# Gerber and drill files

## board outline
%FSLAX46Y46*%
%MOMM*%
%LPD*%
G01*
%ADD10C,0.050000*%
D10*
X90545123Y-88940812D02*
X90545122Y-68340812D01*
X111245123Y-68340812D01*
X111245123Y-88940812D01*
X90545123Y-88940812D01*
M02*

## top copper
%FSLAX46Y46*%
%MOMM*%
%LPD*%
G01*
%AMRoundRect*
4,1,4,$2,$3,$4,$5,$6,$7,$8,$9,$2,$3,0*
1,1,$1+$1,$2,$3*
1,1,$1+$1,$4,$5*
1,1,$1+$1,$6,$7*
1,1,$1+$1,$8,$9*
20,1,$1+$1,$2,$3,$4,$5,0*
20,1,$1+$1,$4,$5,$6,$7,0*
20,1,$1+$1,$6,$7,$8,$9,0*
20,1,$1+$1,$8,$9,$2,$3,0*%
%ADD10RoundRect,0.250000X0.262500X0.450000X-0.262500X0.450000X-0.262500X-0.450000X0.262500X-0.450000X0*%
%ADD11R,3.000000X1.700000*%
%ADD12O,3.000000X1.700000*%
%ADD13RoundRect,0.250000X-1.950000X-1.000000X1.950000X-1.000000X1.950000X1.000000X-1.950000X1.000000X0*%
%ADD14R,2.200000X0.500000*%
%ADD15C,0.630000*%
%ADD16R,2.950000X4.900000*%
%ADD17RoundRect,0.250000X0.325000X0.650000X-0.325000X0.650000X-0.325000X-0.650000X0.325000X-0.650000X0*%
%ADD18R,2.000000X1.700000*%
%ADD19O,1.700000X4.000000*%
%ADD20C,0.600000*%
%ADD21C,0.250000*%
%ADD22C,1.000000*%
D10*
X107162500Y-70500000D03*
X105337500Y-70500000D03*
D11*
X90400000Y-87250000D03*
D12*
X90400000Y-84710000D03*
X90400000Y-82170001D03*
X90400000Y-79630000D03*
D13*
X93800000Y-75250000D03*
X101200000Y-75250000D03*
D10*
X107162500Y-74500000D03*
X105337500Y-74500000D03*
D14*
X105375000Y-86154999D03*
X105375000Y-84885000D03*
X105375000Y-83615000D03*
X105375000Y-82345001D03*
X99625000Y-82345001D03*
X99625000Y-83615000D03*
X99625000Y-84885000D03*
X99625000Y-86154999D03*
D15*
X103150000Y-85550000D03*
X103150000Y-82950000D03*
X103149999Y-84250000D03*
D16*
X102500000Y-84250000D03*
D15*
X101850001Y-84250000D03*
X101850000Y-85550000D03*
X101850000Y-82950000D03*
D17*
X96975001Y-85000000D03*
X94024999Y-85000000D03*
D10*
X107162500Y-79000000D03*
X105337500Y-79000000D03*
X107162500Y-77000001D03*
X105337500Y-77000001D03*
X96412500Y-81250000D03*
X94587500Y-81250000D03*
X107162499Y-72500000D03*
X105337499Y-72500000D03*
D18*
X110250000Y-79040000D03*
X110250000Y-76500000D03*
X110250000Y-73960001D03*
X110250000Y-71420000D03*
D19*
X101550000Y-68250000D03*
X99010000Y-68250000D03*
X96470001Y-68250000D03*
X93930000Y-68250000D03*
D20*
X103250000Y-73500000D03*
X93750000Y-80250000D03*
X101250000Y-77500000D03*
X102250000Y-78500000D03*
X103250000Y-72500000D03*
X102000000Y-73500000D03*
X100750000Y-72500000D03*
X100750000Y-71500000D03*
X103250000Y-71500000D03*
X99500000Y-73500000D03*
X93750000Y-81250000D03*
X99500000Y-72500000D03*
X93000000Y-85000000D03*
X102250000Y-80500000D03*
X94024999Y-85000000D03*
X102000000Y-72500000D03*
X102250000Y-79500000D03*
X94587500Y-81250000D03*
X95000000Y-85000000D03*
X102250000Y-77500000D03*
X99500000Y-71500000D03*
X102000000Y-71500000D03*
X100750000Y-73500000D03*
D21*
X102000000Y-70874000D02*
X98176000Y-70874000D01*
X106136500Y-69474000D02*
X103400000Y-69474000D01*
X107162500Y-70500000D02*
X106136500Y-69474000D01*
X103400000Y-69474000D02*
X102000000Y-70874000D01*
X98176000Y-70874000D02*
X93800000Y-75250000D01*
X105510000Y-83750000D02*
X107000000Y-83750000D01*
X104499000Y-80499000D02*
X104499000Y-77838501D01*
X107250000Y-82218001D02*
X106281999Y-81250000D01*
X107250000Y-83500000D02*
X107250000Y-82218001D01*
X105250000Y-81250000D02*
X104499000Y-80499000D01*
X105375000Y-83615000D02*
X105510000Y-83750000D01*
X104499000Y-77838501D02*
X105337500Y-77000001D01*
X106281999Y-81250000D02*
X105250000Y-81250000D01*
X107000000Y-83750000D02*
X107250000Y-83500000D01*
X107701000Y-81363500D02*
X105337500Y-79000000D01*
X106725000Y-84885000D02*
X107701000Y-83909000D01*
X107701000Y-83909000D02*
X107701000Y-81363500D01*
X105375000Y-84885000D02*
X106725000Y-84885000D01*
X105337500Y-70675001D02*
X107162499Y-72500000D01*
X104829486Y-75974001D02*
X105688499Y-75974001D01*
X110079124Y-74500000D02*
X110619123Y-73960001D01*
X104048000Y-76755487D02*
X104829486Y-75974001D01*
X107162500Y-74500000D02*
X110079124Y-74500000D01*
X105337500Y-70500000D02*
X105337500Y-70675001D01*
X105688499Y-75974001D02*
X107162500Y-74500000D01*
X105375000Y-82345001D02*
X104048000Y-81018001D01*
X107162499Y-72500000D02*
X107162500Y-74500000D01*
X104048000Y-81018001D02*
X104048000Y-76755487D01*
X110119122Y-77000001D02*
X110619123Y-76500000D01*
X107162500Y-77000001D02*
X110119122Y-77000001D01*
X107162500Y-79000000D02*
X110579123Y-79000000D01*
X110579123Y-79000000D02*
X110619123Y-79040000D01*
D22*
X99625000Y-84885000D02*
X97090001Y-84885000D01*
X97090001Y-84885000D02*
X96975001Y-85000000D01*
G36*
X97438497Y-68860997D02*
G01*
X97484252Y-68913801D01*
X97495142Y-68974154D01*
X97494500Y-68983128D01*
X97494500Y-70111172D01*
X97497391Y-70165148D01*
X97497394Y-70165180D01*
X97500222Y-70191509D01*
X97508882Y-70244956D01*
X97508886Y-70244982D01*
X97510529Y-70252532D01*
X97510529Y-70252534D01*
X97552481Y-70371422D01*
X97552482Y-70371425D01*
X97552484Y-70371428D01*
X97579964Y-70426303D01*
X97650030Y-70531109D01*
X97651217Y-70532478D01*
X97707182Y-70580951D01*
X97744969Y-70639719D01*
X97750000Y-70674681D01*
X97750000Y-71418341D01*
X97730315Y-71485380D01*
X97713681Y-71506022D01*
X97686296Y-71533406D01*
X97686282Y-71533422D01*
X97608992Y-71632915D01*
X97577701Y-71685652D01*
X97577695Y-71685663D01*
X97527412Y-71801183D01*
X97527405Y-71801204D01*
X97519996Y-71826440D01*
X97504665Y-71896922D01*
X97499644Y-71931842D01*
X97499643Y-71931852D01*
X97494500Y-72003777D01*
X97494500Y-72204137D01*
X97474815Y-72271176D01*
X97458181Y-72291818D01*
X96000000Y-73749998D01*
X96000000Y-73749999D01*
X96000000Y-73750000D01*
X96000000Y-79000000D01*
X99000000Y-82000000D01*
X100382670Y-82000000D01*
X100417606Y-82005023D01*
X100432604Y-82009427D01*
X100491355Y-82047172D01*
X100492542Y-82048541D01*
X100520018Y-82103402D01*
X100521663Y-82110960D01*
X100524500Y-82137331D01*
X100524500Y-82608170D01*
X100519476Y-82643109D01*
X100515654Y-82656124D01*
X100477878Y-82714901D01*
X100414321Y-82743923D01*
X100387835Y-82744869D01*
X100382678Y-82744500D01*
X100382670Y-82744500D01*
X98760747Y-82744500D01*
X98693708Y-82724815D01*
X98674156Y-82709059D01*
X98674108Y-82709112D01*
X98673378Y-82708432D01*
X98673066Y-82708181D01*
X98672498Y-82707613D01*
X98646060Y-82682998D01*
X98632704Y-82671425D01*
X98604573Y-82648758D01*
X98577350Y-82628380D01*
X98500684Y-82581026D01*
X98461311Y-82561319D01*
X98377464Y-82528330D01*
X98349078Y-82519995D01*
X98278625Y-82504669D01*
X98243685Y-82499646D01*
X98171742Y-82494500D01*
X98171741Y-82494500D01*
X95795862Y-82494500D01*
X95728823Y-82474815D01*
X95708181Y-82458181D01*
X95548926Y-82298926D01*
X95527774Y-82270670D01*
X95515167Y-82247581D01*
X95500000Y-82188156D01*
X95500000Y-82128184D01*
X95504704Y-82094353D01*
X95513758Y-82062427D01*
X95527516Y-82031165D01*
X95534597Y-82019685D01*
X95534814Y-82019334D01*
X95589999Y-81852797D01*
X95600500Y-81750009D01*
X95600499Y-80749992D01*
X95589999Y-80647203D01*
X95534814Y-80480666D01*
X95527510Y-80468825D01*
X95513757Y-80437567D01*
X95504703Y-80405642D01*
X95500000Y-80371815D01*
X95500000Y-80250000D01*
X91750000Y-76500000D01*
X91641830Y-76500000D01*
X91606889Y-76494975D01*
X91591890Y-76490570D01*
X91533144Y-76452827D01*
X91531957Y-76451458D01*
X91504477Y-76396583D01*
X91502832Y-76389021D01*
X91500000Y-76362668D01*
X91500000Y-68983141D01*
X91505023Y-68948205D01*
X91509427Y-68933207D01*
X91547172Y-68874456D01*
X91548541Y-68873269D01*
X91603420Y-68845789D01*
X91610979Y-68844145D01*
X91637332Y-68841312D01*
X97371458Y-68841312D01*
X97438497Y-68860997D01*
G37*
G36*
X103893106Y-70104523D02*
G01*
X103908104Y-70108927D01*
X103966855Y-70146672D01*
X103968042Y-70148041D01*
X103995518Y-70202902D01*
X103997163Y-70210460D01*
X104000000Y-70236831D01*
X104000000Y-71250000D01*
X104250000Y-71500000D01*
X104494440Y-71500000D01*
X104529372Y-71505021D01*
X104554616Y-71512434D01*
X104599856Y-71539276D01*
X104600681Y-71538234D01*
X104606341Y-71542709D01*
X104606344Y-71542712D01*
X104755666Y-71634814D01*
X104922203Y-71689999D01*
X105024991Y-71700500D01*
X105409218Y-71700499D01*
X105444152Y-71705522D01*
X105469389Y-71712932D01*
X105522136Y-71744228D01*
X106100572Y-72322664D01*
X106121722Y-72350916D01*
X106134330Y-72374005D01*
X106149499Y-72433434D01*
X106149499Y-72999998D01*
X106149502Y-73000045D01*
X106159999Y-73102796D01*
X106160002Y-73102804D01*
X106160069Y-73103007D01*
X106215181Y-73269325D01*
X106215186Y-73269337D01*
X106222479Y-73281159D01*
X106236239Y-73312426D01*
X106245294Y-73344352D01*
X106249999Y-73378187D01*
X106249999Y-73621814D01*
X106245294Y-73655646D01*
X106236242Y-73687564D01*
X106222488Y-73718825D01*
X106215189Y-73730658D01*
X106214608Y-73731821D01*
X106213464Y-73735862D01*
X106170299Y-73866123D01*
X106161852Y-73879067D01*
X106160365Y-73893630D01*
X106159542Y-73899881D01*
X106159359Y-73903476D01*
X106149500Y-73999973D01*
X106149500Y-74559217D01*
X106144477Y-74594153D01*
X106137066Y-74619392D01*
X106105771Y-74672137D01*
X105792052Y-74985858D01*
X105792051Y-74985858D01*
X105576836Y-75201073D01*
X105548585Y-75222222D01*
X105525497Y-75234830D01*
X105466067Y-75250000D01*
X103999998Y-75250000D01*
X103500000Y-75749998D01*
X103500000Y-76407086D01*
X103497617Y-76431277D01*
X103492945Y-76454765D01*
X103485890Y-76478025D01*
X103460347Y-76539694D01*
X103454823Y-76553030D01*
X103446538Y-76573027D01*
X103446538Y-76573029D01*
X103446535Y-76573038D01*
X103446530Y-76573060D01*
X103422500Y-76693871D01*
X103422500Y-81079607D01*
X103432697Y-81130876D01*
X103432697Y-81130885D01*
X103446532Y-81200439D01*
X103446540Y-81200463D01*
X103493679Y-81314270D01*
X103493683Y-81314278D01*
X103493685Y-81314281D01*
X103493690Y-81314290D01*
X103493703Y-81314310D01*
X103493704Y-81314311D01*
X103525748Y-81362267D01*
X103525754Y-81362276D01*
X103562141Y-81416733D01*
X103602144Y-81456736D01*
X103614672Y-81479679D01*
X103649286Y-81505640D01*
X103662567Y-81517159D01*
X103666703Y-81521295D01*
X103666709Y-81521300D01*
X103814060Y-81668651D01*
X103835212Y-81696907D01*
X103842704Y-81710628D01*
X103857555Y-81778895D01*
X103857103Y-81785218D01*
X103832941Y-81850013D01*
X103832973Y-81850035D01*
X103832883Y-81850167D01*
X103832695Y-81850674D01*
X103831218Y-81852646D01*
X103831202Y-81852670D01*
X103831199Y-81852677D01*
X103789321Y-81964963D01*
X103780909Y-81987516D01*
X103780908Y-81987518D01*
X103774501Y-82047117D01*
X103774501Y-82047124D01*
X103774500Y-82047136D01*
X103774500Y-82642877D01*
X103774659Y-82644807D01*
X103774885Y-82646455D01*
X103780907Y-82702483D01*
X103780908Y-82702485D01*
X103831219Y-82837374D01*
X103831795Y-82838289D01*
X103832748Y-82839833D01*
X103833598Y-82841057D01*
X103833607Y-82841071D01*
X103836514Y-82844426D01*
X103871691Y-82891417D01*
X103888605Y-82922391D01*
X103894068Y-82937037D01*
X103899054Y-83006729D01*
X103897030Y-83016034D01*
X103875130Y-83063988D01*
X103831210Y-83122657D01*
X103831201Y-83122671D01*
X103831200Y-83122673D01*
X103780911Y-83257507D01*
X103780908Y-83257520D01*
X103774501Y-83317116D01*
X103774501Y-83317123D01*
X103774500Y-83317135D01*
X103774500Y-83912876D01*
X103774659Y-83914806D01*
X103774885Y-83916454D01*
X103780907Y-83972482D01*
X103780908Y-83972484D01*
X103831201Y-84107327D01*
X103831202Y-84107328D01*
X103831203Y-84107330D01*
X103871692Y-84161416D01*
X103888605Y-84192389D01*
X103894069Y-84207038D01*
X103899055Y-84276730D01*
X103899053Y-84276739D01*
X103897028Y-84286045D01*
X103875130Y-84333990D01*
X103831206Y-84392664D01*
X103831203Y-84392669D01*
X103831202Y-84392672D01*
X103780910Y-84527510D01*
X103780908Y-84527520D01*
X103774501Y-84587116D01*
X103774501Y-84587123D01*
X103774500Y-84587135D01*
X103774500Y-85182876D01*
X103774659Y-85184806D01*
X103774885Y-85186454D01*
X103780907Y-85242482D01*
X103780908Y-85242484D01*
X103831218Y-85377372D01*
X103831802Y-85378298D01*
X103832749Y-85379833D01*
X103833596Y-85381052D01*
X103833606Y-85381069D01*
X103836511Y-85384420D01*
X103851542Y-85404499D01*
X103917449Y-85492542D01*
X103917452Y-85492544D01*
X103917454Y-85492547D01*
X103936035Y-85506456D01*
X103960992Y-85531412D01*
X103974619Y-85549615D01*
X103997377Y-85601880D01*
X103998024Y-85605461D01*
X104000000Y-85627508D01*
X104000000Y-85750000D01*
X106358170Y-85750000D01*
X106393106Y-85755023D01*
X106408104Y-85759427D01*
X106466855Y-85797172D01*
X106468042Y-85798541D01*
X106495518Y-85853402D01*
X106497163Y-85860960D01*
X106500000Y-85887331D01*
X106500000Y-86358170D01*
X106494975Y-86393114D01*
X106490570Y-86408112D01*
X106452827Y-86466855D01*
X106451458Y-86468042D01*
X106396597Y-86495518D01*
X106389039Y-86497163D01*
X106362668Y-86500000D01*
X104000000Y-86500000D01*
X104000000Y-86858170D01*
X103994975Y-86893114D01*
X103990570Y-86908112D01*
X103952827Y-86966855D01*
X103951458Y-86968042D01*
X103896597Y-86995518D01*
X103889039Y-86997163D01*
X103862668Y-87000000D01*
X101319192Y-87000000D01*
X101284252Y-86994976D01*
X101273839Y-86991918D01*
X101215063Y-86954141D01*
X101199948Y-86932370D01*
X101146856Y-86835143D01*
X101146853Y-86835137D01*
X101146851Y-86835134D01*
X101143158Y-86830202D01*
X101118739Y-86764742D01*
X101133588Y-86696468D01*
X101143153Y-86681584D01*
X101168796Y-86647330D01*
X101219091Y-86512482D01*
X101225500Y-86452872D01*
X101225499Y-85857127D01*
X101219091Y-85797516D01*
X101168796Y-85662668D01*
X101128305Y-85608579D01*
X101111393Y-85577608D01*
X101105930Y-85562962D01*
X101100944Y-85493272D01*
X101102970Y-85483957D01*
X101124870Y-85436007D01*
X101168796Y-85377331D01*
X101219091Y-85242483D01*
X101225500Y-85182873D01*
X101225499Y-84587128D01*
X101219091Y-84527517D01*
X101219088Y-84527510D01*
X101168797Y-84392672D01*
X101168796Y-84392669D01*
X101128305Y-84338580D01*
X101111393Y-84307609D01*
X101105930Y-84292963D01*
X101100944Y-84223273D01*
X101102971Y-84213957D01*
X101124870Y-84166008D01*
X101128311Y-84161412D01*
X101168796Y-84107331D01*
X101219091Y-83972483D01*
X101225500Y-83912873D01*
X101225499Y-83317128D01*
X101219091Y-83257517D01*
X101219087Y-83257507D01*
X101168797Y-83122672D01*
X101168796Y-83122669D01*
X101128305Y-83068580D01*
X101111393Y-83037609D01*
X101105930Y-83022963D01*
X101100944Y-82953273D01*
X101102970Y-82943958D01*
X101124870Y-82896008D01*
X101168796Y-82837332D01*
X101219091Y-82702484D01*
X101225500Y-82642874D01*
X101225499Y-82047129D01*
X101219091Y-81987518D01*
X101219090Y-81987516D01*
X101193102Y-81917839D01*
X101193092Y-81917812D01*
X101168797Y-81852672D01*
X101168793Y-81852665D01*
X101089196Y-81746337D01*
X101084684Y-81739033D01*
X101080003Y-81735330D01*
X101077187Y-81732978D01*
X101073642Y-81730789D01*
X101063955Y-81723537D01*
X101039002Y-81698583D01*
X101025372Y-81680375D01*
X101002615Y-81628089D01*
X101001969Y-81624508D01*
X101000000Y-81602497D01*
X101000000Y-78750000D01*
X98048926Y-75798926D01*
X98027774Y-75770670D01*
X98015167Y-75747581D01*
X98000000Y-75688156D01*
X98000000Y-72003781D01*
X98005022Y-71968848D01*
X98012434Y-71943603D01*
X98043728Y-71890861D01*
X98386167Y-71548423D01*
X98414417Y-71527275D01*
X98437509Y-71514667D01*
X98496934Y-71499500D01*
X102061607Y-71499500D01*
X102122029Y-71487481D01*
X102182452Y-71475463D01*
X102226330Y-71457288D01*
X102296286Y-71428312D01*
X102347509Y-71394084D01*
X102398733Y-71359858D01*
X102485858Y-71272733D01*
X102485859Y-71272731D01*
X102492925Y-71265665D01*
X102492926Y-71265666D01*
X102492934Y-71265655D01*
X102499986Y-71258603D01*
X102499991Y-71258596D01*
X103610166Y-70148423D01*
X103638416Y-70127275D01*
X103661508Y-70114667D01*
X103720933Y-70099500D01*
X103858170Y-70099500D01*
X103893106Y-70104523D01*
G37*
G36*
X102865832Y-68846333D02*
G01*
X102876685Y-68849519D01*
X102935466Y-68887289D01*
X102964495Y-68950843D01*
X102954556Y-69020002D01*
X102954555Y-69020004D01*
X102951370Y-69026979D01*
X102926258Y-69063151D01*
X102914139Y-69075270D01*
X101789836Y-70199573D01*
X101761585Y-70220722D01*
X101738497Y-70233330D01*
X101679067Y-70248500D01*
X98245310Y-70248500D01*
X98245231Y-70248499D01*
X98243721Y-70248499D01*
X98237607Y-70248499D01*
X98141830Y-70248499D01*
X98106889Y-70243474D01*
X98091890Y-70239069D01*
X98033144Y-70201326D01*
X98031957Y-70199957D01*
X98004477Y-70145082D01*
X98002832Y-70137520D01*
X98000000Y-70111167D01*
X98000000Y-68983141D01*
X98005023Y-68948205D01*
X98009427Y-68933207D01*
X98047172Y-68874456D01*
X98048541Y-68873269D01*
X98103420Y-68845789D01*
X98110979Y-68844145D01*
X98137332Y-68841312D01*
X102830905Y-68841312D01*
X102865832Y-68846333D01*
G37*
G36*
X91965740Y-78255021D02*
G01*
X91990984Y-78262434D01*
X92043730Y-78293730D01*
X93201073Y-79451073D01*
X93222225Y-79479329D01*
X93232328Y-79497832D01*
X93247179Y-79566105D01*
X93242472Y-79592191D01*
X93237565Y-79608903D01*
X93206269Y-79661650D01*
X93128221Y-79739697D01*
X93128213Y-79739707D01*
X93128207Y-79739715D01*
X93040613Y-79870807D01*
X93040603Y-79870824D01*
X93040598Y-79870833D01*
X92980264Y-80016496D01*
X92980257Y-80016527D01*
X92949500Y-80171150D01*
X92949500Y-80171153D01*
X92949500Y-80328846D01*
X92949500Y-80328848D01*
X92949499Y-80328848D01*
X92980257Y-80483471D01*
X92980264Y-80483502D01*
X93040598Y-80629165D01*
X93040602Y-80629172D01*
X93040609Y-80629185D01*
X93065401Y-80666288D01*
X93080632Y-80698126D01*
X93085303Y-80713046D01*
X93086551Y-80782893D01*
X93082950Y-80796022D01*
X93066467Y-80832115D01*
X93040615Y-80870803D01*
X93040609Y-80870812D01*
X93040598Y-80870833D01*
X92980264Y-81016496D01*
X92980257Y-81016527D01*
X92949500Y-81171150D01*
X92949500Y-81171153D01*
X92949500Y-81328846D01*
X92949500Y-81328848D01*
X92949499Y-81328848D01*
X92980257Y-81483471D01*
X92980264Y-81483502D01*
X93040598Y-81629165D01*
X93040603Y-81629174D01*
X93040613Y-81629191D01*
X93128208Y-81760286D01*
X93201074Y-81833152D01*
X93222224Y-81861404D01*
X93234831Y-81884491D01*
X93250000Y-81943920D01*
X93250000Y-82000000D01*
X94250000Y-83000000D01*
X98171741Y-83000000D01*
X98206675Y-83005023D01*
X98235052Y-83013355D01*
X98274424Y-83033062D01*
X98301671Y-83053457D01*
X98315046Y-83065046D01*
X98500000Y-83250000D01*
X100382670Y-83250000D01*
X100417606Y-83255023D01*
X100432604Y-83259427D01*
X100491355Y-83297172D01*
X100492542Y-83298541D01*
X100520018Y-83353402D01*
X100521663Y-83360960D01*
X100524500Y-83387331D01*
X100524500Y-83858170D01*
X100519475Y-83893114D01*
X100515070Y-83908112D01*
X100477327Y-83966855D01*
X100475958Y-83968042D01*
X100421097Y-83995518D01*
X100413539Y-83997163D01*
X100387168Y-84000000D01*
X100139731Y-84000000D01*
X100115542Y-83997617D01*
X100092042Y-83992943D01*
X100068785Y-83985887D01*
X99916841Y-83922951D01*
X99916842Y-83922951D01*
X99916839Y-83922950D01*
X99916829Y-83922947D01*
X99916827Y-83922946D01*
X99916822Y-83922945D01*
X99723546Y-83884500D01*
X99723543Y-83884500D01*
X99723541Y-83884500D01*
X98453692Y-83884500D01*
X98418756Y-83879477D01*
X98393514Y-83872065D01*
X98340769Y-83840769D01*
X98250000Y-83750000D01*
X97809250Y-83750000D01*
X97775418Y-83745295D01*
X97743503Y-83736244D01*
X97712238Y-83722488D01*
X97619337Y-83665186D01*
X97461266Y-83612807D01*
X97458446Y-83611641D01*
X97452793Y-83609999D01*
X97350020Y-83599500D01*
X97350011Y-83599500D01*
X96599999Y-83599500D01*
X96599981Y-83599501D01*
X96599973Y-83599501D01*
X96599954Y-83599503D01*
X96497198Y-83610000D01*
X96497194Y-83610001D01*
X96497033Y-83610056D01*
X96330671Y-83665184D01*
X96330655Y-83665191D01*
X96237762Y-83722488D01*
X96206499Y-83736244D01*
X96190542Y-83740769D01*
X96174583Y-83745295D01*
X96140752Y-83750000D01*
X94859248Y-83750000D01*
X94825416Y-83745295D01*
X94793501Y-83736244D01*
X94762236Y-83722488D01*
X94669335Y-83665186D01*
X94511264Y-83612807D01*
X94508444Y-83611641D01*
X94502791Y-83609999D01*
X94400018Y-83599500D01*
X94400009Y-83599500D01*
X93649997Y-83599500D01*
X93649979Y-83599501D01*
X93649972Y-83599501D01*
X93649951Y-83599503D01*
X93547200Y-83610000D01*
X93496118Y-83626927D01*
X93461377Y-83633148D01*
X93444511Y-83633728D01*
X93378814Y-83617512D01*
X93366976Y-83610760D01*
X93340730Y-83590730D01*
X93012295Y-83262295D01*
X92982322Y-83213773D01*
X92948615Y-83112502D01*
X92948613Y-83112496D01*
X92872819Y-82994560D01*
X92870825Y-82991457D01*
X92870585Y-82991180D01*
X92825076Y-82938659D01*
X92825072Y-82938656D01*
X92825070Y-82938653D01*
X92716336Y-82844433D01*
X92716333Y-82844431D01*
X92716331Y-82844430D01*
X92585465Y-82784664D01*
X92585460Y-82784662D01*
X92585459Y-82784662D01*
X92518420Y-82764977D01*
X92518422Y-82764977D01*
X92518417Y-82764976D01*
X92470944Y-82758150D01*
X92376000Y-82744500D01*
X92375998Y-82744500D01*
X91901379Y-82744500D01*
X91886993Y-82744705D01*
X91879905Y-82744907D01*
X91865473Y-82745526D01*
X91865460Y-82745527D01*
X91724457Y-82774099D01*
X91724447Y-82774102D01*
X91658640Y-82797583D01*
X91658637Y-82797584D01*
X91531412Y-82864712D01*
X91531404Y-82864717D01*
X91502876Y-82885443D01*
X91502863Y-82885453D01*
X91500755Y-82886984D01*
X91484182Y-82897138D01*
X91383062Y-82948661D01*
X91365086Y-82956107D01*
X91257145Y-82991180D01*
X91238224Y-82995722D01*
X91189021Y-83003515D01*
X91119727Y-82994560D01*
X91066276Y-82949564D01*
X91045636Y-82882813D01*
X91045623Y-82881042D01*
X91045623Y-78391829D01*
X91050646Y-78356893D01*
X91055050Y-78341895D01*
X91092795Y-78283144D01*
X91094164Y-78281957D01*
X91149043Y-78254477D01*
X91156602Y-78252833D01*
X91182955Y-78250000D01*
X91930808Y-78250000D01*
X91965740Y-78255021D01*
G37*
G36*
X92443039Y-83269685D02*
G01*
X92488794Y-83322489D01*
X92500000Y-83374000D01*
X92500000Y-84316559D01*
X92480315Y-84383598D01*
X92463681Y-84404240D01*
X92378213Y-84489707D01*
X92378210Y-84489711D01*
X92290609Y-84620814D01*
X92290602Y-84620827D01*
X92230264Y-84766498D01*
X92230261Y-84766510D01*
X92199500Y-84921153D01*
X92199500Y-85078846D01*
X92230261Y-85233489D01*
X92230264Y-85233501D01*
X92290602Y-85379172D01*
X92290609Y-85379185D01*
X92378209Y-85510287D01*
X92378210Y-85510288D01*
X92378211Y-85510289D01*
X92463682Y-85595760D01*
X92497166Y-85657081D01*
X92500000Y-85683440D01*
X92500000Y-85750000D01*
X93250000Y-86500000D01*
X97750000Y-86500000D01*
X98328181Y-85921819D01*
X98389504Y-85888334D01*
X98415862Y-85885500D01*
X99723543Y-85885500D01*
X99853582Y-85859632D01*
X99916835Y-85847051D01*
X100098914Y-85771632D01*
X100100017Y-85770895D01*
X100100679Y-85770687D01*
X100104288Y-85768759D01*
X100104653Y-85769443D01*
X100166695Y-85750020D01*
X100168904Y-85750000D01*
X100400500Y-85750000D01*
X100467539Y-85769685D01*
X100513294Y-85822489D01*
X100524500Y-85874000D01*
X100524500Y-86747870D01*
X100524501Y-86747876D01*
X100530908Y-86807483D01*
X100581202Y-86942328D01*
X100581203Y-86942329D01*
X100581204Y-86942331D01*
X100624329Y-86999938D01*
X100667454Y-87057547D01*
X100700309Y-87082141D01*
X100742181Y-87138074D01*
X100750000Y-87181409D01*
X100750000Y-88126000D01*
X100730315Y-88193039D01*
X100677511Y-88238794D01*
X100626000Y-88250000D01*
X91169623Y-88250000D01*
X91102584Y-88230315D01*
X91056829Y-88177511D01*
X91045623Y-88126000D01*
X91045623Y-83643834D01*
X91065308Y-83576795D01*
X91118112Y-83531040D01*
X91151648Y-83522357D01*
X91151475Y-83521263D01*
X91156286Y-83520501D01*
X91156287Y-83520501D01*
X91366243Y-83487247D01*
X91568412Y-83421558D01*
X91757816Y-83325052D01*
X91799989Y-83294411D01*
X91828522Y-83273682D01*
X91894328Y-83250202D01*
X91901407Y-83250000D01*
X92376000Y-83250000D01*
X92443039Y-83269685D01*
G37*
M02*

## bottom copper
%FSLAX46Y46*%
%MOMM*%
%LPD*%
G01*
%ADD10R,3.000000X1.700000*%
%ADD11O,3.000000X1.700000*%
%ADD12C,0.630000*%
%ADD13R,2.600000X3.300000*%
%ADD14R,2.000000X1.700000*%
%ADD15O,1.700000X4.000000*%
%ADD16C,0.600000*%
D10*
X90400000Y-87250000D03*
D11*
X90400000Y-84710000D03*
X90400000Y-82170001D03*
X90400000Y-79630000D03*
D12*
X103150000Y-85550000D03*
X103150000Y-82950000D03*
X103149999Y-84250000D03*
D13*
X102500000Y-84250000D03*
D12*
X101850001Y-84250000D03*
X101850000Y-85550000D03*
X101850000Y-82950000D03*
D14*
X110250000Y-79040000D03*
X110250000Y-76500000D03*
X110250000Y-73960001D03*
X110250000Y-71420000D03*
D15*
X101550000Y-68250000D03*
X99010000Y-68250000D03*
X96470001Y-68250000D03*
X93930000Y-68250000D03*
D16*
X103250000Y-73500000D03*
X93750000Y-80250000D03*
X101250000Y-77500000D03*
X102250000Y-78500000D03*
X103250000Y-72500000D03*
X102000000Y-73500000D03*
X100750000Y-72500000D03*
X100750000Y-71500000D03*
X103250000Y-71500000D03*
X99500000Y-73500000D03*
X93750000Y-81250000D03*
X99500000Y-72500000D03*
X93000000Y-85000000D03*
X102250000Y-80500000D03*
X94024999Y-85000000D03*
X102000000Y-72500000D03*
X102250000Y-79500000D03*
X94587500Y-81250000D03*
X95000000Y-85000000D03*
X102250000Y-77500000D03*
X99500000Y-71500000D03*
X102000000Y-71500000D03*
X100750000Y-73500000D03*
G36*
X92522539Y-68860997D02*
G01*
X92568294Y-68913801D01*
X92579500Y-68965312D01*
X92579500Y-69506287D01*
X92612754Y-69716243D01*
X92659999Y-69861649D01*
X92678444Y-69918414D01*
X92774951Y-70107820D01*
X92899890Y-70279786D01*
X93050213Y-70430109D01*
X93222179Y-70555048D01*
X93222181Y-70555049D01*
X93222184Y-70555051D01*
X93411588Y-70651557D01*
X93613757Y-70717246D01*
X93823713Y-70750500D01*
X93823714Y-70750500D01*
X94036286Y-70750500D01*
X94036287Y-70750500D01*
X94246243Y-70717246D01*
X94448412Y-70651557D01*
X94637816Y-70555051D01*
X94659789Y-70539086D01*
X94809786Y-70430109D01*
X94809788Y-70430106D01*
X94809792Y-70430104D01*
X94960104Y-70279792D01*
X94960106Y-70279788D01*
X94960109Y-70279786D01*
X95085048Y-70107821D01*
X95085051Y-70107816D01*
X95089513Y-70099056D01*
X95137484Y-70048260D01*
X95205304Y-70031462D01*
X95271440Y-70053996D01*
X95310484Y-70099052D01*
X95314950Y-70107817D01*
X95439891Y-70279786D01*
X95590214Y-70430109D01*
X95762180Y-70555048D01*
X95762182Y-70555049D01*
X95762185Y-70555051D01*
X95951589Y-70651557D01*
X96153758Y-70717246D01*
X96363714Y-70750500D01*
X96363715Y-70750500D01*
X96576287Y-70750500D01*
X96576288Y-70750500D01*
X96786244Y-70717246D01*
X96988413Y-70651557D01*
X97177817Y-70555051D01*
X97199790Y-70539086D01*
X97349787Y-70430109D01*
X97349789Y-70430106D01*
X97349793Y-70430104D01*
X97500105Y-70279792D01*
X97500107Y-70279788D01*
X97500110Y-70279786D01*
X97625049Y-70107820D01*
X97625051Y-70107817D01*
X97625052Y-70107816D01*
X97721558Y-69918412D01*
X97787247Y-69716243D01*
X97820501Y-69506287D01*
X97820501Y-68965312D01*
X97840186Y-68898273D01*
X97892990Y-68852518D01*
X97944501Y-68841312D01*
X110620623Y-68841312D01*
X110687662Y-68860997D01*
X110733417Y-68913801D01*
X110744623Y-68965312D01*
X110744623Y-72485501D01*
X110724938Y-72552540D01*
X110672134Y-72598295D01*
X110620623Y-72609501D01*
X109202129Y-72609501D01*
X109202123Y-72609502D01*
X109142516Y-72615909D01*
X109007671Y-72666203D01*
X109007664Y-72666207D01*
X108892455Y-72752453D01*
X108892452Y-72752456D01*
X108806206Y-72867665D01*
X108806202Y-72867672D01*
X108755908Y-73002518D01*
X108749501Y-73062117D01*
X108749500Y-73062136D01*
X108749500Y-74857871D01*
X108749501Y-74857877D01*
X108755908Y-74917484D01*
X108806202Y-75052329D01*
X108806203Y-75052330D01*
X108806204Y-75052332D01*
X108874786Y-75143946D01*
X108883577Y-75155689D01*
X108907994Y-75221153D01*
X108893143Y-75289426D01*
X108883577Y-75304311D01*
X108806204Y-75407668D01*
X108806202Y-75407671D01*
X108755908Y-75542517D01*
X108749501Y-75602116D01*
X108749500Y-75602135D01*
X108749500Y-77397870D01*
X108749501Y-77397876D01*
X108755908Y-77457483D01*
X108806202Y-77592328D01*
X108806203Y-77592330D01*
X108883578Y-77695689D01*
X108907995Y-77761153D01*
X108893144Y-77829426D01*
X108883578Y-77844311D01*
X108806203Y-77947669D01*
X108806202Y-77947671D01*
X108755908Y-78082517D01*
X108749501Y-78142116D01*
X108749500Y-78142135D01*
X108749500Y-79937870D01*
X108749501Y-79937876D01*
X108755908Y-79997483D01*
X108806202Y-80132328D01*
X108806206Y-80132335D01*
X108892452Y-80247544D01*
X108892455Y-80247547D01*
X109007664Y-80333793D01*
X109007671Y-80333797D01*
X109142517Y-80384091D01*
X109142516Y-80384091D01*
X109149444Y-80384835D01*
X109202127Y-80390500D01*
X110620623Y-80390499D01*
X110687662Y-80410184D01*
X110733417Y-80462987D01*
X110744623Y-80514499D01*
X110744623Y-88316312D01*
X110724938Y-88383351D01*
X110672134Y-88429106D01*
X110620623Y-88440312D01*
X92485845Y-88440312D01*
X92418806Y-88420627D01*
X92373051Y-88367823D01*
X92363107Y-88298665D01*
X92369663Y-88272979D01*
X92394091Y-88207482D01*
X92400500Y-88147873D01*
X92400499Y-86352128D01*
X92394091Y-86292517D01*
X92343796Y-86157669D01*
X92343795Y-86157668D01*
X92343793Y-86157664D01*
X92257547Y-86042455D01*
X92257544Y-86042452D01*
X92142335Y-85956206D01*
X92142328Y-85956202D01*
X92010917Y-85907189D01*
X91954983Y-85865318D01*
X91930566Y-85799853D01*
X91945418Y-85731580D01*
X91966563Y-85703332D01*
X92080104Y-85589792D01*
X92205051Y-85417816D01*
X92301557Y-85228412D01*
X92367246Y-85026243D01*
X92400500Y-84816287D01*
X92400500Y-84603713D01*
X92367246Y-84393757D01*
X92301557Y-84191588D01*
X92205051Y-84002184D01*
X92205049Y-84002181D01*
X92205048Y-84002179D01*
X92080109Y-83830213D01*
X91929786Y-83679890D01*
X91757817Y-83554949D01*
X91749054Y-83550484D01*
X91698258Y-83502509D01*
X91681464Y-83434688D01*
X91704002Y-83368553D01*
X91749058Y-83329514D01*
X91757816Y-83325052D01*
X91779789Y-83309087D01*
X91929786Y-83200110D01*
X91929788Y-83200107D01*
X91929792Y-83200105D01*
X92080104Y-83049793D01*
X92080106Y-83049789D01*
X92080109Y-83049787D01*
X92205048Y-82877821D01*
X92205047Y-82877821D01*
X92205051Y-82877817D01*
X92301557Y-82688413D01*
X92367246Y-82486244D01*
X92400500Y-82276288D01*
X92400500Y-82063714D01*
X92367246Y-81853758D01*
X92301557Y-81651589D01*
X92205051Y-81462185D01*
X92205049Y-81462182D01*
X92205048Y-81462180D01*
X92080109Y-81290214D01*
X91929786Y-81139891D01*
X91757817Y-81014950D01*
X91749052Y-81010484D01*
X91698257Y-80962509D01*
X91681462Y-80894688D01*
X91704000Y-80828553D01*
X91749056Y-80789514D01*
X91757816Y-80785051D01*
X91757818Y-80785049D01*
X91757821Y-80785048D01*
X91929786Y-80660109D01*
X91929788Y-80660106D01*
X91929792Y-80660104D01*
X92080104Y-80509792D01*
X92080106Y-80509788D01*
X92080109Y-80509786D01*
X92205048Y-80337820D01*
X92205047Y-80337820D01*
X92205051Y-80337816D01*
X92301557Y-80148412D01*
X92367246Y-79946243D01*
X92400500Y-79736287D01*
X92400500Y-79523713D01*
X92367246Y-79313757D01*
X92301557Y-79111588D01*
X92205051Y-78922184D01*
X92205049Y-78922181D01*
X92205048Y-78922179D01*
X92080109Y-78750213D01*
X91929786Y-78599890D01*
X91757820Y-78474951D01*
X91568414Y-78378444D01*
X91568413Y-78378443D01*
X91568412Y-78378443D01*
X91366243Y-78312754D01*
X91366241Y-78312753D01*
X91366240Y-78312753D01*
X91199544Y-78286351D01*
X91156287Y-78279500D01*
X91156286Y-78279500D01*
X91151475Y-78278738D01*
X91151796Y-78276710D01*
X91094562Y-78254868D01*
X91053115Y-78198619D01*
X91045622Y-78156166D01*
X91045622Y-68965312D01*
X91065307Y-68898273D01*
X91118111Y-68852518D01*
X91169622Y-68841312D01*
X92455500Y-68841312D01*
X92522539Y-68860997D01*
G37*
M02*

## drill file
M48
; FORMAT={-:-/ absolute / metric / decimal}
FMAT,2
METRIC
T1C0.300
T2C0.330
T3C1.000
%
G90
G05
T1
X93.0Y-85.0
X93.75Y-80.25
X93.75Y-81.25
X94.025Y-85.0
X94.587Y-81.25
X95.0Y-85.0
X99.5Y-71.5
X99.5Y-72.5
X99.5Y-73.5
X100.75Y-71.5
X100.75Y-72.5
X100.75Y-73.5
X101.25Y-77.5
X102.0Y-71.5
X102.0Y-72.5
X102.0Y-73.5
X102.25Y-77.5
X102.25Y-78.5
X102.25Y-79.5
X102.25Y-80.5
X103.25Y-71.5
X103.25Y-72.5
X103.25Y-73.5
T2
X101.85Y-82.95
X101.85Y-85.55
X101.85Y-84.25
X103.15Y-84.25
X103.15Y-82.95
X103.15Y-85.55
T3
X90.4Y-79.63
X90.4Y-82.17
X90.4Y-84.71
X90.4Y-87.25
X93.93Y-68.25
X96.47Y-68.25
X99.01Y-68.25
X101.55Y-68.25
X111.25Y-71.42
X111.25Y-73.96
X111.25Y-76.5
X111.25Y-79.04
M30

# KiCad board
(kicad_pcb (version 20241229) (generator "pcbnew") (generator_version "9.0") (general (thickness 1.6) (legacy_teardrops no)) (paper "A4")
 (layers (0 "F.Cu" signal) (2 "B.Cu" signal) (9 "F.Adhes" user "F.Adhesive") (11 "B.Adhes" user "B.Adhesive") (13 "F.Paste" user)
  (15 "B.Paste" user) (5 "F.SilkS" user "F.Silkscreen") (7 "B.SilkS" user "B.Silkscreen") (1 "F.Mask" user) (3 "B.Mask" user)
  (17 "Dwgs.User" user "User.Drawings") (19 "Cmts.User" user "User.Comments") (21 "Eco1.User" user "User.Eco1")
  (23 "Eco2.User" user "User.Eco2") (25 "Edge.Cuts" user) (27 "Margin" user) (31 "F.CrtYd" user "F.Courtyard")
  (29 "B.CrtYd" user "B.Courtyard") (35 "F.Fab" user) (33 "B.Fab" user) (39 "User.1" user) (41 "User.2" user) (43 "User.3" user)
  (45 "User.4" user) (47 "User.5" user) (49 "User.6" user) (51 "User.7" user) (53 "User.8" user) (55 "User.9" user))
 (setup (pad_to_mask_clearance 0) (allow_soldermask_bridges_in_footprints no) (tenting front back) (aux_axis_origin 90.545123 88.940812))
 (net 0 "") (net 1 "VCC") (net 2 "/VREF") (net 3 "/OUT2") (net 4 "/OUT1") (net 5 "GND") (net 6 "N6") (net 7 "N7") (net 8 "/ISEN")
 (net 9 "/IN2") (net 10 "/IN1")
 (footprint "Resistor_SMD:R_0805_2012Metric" (layer "F.Cu") (at 106.25 70.5 180)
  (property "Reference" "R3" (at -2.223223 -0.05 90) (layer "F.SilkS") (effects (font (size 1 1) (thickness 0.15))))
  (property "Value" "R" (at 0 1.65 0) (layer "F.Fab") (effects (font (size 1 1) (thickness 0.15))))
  (pad "1" smd roundrect (at -0.9125 0 180) (size 1.025 1.4) (layers "F.Cu" "F.Mask" "F.Paste") (roundrect_rratio 0.243902) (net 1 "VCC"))
  (pad "2" smd roundrect (at 0.9125 0 180) (size 1.025 1.4) (layers "F.Cu" "F.Mask" "F.Paste") (roundrect_rratio 0.243902) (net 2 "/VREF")))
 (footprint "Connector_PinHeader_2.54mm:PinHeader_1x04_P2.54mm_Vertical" (layer "F.Cu") (at 90.4 87.25 180)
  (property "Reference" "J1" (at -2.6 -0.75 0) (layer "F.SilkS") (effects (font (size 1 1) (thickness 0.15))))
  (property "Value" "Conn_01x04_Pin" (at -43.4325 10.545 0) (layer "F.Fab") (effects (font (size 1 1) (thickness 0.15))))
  (pad "1" thru_hole rect (at 0 0 180) (size 3 1.7) (drill 1) (layers "*.Cu" "*.Mask") (remove_unused_layers no) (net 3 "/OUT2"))
  (pad "2" thru_hole oval (at 0 2.54 180) (size 3 1.7) (drill 1) (layers "*.Cu" "*.Mask") (remove_unused_layers no) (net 3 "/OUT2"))
  (pad "3" thru_hole oval (at 0 5.079999 180) (size 3 1.7) (drill 1) (layers "*.Cu" "*.Mask") (remove_unused_layers no) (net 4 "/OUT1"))
  (pad "4" thru_hole oval (at 0 7.62 180) (size 3 1.7) (drill 1) (layers "*.Cu" "*.Mask") (remove_unused_layers no) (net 4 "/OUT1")))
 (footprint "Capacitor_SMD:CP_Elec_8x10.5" (layer "F.Cu") (at 97.5 75.25)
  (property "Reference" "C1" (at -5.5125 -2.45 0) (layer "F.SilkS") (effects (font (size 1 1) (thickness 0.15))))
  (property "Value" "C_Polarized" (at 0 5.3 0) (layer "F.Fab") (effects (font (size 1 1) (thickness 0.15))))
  (pad "1" smd roundrect (at -3.7 0) (size 4.4 2.5) (layers "F.Cu" "F.Mask" "F.Paste") (roundrect_rratio 0.1) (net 1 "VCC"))
  (pad "2" smd roundrect (at 3.7 0) (size 4.4 2.5) (layers "F.Cu" "F.Mask" "F.Paste") (roundrect_rratio 0.1) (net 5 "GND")))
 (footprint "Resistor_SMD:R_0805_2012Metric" (layer "F.Cu") (at 106.25 74.5 180)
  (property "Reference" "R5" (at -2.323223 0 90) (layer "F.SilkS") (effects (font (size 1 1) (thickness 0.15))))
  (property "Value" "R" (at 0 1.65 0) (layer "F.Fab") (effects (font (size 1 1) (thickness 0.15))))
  (pad "1" smd roundrect (at -0.9125 0 180) (size 1.025 1.4) (layers "F.Cu" "F.Mask" "F.Paste") (roundrect_rratio 0.243902) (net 2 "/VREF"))
  (pad "2" smd roundrect (at 0.9125 0 180) (size 1.025 1.4) (layers "F.Cu" "F.Mask" "F.Paste") (roundrect_rratio 0.243902) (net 5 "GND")))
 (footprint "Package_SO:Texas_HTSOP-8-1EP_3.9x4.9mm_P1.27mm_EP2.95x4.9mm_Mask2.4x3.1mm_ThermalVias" (layer "F.Cu") (at 102.5 84.25 180)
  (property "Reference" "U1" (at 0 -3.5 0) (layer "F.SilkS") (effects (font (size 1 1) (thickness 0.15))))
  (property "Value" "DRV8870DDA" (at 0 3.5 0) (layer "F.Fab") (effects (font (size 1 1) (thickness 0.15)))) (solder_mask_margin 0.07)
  (pad "" smd rect (at 0 0 180) (size 2.4 3.1) (layers "F.Mask"))
  (pad "" smd rect (at 0 0 180) (size 2.4 3.1) (layers "F.Paste"))
  (pad "1" smd rect (at -2.875 -1.904999 180) (size 2.2 0.5) (layers "F.Cu" "F.Mask" "F.Paste") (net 5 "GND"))
  (pad "2" smd rect (at -2.875 -0.635 180) (size 2.2 0.5) (layers "F.Cu" "F.Mask" "F.Paste") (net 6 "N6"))
  (pad "3" smd rect (at -2.875 0.635 180) (size 2.2 0.5) (layers "F.Cu" "F.Mask" "F.Paste") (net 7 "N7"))
  (pad "4" smd rect (at -2.875 1.904999 180) (size 2.2 0.5) (layers "F.Cu" "F.Mask" "F.Paste") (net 2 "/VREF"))
  (pad "5" smd rect (at 2.875 1.904999 180) (size 2.2 0.5) (layers "F.Cu" "F.Mask" "F.Paste") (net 1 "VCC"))
  (pad "6" smd rect (at 2.875 0.635 180) (size 2.2 0.5) (layers "F.Cu" "F.Mask" "F.Paste") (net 4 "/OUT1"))
  (pad "7" smd rect (at 2.875 -0.635 180) (size 2.2 0.5) (layers "F.Cu" "F.Mask" "F.Paste") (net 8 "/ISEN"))
  (pad "8" smd rect (at 2.875 -1.904999 180) (size 2.2 0.5) (layers "F.Cu" "F.Mask" "F.Paste") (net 3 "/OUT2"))
  (pad "9" thru_hole circle (at -0.65 -1.3 180) (size 0.63 0.63) (drill 0.33) (layers "*.Cu" "*.Mask") (remove_unused_layers no)
   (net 5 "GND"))
  (pad "9" thru_hole circle (at -0.65 1.3 180) (size 0.63 0.63) (drill 0.33) (layers "*.Cu" "*.Mask") (remove_unused_layers no)
   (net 5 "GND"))
  (pad "9" thru_hole circle (at -0.649999 0 180) (size 0.63 0.63) (drill 0.33) (layers "*.Cu" "*.Mask") (remove_unused_layers no)
   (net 5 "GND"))
  (pad "9" smd rect (at 0 0 180) (size 2.6 3.3) (layers "B.Cu") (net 5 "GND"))
  (pad "9" smd rect (at 0 0 180) (size 2.95 4.9) (layers "F.Cu") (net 5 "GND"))
  (pad "9" thru_hole circle (at 0.649999 0 180) (size 0.63 0.63) (drill 0.33) (layers "*.Cu" "*.Mask") (remove_unused_layers no)
   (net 5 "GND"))
  (pad "9" thru_hole circle (at 0.65 -1.3 180) (size 0.63 0.63) (drill 0.33) (layers "*.Cu" "*.Mask") (remove_unused_layers no)
   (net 5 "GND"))
  (pad "9" thru_hole circle (at 0.65 1.3 180) (size 0.63 0.63) (drill 0.33) (layers "*.Cu" "*.Mask") (remove_unused_layers no) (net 5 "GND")))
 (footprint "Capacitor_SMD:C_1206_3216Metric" (layer "F.Cu") (at 95.5 85 180)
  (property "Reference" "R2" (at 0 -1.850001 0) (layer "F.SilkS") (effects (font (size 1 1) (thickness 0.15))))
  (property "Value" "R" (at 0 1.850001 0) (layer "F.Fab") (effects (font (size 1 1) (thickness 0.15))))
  (pad "1" smd roundrect (at -1.475001 0 180) (size 1.15 1.8) (layers "F.Cu" "F.Mask" "F.Paste") (roundrect_rratio 0.217391) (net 8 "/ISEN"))
  (pad "2" smd roundrect (at 1.475001 0 180) (size 1.15 1.8) (layers "F.Cu" "F.Mask" "F.Paste") (roundrect_rratio 0.217391) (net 5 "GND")))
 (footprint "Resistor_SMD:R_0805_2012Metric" (layer "F.Cu") (at 106.25 79 180)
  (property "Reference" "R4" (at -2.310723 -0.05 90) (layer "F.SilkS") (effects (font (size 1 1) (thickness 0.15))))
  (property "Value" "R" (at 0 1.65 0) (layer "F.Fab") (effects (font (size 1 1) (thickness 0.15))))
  (pad "1" smd roundrect (at -0.9125 0 180) (size 1.025 1.4) (layers "F.Cu" "F.Mask" "F.Paste") (roundrect_rratio 0.243902) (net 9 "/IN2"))
  (pad "2" smd roundrect (at 0.9125 0 180) (size 1.025 1.4) (layers "F.Cu" "F.Mask" "F.Paste") (roundrect_rratio 0.243902) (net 6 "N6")))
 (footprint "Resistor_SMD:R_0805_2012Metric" (layer "F.Cu") (at 106.25 77.000001 180)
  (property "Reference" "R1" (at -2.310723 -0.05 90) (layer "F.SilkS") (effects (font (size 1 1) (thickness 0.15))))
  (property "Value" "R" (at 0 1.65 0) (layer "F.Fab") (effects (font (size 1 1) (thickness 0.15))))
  (pad "1" smd roundrect (at -0.9125 0 180) (size 1.025 1.4) (layers "F.Cu" "F.Mask" "F.Paste") (roundrect_rratio 0.243902) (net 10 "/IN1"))
  (pad "2" smd roundrect (at 0.9125 0 180) (size 1.025 1.4) (layers "F.Cu" "F.Mask" "F.Paste") (roundrect_rratio 0.243902) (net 7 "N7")))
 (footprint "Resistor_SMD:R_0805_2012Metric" (layer "F.Cu") (at 95.5 81.25 180)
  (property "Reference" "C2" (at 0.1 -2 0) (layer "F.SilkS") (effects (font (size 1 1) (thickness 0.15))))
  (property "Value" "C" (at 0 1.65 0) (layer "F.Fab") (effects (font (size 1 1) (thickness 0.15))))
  (pad "1" smd roundrect (at -0.9125 0 180) (size 1.025 1.4) (layers "F.Cu" "F.Mask" "F.Paste") (roundrect_rratio 0.243902) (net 1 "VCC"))
  (pad "2" smd roundrect (at 0.9125 0 180) (size 1.025 1.4) (layers "F.Cu" "F.Mask" "F.Paste") (roundrect_rratio 0.243902) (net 5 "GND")))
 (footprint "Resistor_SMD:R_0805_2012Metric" (layer "F.Cu") (at 106.249999 72.5 180)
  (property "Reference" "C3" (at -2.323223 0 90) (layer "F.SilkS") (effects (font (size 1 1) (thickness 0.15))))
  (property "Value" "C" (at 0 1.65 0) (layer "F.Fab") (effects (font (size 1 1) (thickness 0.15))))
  (pad "1" smd roundrect (at -0.9125 0 180) (size 1.025 1.4) (layers "F.Cu" "F.Mask" "F.Paste") (roundrect_rratio 0.243902) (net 2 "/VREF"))
  (pad "2" smd roundrect (at 0.9125 0 180) (size 1.025 1.4) (layers "F.Cu" "F.Mask" "F.Paste") (roundrect_rratio 0.243902) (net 5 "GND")))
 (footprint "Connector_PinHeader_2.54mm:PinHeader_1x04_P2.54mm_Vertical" (layer "F.Cu") (at 111.25 79.04 180)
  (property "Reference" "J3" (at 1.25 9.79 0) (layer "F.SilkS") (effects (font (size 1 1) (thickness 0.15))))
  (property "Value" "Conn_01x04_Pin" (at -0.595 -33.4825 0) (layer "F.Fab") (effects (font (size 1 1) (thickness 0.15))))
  (pad "1" thru_hole rect (at 0 0 180) (size 2 1.7) (drill 1 (offset 1 0)) (layers "*.Cu" "*.Mask") (remove_unused_layers no) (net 9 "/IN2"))
  (pad "2" thru_hole rect (at 0 2.54 180) (size 2 1.7) (drill 1 (offset 1 0)) (layers "*.Cu" "*.Mask") (remove_unused_layers no)
   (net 10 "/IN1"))
  (pad "3" thru_hole rect (at 0 5.079999 180) (size 2 1.7) (drill 1 (offset 1 0)) (layers "*.Cu" "*.Mask") (remove_unused_layers no)
   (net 2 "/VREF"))
  (pad "4" thru_hole rect (at 0 7.62 180) (size 2 1.7) (drill 1 (offset 1 0)) (layers "*.Cu" "*.Mask") (remove_unused_layers no)
   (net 5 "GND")))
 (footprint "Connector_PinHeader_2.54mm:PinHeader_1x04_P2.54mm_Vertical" (layer "F.Cu") (at 101.55 68.25 -90)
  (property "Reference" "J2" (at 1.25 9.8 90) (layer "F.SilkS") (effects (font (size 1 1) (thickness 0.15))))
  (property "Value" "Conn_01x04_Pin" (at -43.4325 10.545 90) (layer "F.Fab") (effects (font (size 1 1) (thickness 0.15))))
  (pad "1" thru_hole oval (at 0 0 270) (size 4 1.7) (drill 1) (layers "*.Cu" "*.Mask") (remove_unused_layers no) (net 5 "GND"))
  (pad "2" thru_hole oval (at 0 2.54 270) (size 4 1.7) (drill 1) (layers "*.Cu" "*.Mask") (remove_unused_layers no) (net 5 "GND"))
  (pad "3" thru_hole oval (at 0 5.079999 270) (size 4 1.7) (drill 1) (layers "*.Cu" "*.Mask") (remove_unused_layers no) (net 1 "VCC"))
  (pad "4" thru_hole oval (at 0 7.62 270) (size 4 1.7) (drill 1) (layers "*.Cu" "*.Mask") (remove_unused_layers no) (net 1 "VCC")))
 (gr_poly
  (pts (xy 90.545123 88.940812) (xy 90.545122 68.340812) (xy 111.245123 68.340812) (xy 111.245123 88.940812))
  (stroke (width 0.05) (type default)) (fill no) (layer "Edge.Cuts"))
 (segment (start 102 70.874) (end 98.176 70.874) (width 0.25) (layer "F.Cu") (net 1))
 (segment (start 106.1365 69.474) (end 103.4 69.474) (width 0.25) (layer "F.Cu") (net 1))
 (segment (start 107.1625 70.5) (end 106.1365 69.474) (width 0.25) (layer "F.Cu") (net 1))
 (segment (start 103.4 69.474) (end 102 70.874) (width 0.25) (layer "F.Cu") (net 1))
 (segment (start 98.176 70.874) (end 93.8 75.25) (width 0.25) (layer "F.Cu") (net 1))
 (via (at 103.25 73.5) (size 0.6) (drill 0.3) (layers "F.Cu" "B.Cu") (free yes) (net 5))
 (via (at 93.75 80.25) (size 0.6) (drill 0.3) (layers "F.Cu" "B.Cu") (free yes) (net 5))
 (via (at 101.25 77.5) (size 0.6) (drill 0.3) (layers "F.Cu" "B.Cu") (free yes) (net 5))
 (via (at 102.25 78.5) (size 0.6) (drill 0.3) (layers "F.Cu" "B.Cu") (free yes) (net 5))
 (via (at 103.25 72.5) (size 0.6) (drill 0.3) (layers "F.Cu" "B.Cu") (free yes) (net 5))
 (via (at 102 73.5) (size 0.6) (drill 0.3) (layers "F.Cu" "B.Cu") (free yes) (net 5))
 (via (at 100.75 72.5) (size 0.6) (drill 0.3) (layers "F.Cu" "B.Cu") (free yes) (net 5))
 (via (at 100.75 71.5) (size 0.6) (drill 0.3) (layers "F.Cu" "B.Cu") (free yes) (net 5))
 (via (at 103.25 71.5) (size 0.6) (drill 0.3) (layers "F.Cu" "B.Cu") (free yes) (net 5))
 (via (at 99.5 73.5) (size 0.6) (drill 0.3) (layers "F.Cu" "B.Cu") (free yes) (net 5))
 (via (at 93.75 81.25) (size 0.6) (drill 0.3) (layers "F.Cu" "B.Cu") (free yes) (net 5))
 (via (at 99.5 72.5) (size 0.6) (drill 0.3) (layers "F.Cu" "B.Cu") (free yes) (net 5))
 (via (at 93 85) (size 0.6) (drill 0.3) (layers "F.Cu" "B.Cu") (free yes) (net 5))
 (via (at 102.25 80.5) (size 0.6) (drill 0.3) (layers "F.Cu" "B.Cu") (free yes) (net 5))
 (via (at 94.024999 85) (size 0.6) (drill 0.3) (layers "F.Cu" "B.Cu") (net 5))
 (via (at 102 72.5) (size 0.6) (drill 0.3) (layers "F.Cu" "B.Cu") (free yes) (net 5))
 (via (at 102.25 79.5) (size 0.6) (drill 0.3) (layers "F.Cu" "B.Cu") (free yes) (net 5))
 (via (at 94.5875 81.25) (size 0.6) (drill 0.3) (layers "F.Cu" "B.Cu") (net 5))
 (via (at 95 85) (size 0.6) (drill 0.3) (layers "F.Cu" "B.Cu") (free yes) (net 5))
 (via (at 102.25 77.5) (size 0.6) (drill 0.3) (layers "F.Cu" "B.Cu") (free yes) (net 5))
 (via (at 99.5 71.5) (size 0.6) (drill 0.3) (layers "F.Cu" "B.Cu") (free yes) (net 5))
 (via (at 102 71.5) (size 0.6) (drill 0.3) (layers "F.Cu" "B.Cu") (free yes) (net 5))
 (via (at 100.75 73.5) (size 0.6) (drill 0.3) (layers "F.Cu" "B.Cu") (free yes) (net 5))
 (segment (start 105.51 83.75) (end 107 83.75) (width 0.25) (layer "F.Cu") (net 7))
 (segment (start 104.499 80.499) (end 104.499 77.838501) (width 0.25) (layer "F.Cu") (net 7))
 (segment (start 107.25 82.218001) (end 106.281999 81.25) (width 0.25) (layer "F.Cu") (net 7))
 (segment (start 107.25 83.5) (end 107.25 82.218001) (width 0.25) (layer "F.Cu") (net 7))
 (segment (start 105.25 81.25) (end 104.499 80.499) (width 0.25) (layer "F.Cu") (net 7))
 (segment (start 105.375 83.615) (end 105.51 83.75) (width 0.25) (layer "F.Cu") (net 7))
 (segment (start 104.499 77.838501) (end 105.3375 77.000001) (width 0.25) (layer "F.Cu") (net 7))
 (segment (start 106.281999 81.25) (end 105.25 81.25) (width 0.25) (layer "F.Cu") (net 7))
 (segment (start 107 83.75) (end 107.25 83.5) (width 0.25) (layer "F.Cu") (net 7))
 (segment (start 107.701 81.3635) (end 105.3375 79) (width 0.25) (layer "F.Cu") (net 6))
 (segment (start 106.725 84.885) (end 107.701 83.909) (width 0.25) (layer "F.Cu") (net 6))
 (segment (start 107.701 83.909) (end 107.701 81.3635) (width 0.25) (layer "F.Cu") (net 6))
 (segment (start 105.375 84.885) (end 106.725 84.885) (width 0.25) (layer "F.Cu") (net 6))
 (segment (start 105.3375 70.675001) (end 107.162499 72.5) (width 0.25) (layer "F.Cu") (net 2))
 (segment (start 104.829486 75.974001) (end 105.688499 75.974001) (width 0.25) (layer "F.Cu") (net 2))
 (segment (start 110.079124 74.5) (end 110.619123 73.960001) (width 0.25) (layer "F.Cu") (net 2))
 (segment (start 104.048 76.755487) (end 104.829486 75.974001) (width 0.25) (layer "F.Cu") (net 2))
 (segment (start 107.1625 74.5) (end 110.079124 74.5) (width 0.25) (layer "F.Cu") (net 2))
 (segment (start 105.3375 70.5) (end 105.3375 70.675001) (width 0.25) (layer "F.Cu") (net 2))
 (segment (start 105.688499 75.974001) (end 107.1625 74.5) (width 0.25) (layer "F.Cu") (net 2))
 (segment (start 105.375 82.345001) (end 104.048 81.018001) (width 0.25) (layer "F.Cu") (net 2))
 (segment (start 107.162499 72.5) (end 107.1625 74.5) (width 0.25) (layer "F.Cu") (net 2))
 (segment (start 104.048 81.018001) (end 104.048 76.755487) (width 0.25) (layer "F.Cu") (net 2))
 (segment (start 110.119122 77.000001) (end 110.619123 76.5) (width 0.25) (layer "F.Cu") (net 10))
 (segment (start 107.1625 77.000001) (end 110.119122 77.000001) (width 0.25) (layer "F.Cu") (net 10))
 (segment (start 107.1625 79) (end 110.579123 79) (width 0.25) (layer "F.Cu") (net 9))
 (segment (start 110.579123 79) (end 110.619123 79.04) (width 0.25) (layer "F.Cu") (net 9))
 (segment (start 99.625 84.885) (end 97.090001 84.885) (width 1) (layer "F.Cu") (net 8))
 (segment (start 97.090001 84.885) (end 96.975001 85) (width 1) (layer "F.Cu") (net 8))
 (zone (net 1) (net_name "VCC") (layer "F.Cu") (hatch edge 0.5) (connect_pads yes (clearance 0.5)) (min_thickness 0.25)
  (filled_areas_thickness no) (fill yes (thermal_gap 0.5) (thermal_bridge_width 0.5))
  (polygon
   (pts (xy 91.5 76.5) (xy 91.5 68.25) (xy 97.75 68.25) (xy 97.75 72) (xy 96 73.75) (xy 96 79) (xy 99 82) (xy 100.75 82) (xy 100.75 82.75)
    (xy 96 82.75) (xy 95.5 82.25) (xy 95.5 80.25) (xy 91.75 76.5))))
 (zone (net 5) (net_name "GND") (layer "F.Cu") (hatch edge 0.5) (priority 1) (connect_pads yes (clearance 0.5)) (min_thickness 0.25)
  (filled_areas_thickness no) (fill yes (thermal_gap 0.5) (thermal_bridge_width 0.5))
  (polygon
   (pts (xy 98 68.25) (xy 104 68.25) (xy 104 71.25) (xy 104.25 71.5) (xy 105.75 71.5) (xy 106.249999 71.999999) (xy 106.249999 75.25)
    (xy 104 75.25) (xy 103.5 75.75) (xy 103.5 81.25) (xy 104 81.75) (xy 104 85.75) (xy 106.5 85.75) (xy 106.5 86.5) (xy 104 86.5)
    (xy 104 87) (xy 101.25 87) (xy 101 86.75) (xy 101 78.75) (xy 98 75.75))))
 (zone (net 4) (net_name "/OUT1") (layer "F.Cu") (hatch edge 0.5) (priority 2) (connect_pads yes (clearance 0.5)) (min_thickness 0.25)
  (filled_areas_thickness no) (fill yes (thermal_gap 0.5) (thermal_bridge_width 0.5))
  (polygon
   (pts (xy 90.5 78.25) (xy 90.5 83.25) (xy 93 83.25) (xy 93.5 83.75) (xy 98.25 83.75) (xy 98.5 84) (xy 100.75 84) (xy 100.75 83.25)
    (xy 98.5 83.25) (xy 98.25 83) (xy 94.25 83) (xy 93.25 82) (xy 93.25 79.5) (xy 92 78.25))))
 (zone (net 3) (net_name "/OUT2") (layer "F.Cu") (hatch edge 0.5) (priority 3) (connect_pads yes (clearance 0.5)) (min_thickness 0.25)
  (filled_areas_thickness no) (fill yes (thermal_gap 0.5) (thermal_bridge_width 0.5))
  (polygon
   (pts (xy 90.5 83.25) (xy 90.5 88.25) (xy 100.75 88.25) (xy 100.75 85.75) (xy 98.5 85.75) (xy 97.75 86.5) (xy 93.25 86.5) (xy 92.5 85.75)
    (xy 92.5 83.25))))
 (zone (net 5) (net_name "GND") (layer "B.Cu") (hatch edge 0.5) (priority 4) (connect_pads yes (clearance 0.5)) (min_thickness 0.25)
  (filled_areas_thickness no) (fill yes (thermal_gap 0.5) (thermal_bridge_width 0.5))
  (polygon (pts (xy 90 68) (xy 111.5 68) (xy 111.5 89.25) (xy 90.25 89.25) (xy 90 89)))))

